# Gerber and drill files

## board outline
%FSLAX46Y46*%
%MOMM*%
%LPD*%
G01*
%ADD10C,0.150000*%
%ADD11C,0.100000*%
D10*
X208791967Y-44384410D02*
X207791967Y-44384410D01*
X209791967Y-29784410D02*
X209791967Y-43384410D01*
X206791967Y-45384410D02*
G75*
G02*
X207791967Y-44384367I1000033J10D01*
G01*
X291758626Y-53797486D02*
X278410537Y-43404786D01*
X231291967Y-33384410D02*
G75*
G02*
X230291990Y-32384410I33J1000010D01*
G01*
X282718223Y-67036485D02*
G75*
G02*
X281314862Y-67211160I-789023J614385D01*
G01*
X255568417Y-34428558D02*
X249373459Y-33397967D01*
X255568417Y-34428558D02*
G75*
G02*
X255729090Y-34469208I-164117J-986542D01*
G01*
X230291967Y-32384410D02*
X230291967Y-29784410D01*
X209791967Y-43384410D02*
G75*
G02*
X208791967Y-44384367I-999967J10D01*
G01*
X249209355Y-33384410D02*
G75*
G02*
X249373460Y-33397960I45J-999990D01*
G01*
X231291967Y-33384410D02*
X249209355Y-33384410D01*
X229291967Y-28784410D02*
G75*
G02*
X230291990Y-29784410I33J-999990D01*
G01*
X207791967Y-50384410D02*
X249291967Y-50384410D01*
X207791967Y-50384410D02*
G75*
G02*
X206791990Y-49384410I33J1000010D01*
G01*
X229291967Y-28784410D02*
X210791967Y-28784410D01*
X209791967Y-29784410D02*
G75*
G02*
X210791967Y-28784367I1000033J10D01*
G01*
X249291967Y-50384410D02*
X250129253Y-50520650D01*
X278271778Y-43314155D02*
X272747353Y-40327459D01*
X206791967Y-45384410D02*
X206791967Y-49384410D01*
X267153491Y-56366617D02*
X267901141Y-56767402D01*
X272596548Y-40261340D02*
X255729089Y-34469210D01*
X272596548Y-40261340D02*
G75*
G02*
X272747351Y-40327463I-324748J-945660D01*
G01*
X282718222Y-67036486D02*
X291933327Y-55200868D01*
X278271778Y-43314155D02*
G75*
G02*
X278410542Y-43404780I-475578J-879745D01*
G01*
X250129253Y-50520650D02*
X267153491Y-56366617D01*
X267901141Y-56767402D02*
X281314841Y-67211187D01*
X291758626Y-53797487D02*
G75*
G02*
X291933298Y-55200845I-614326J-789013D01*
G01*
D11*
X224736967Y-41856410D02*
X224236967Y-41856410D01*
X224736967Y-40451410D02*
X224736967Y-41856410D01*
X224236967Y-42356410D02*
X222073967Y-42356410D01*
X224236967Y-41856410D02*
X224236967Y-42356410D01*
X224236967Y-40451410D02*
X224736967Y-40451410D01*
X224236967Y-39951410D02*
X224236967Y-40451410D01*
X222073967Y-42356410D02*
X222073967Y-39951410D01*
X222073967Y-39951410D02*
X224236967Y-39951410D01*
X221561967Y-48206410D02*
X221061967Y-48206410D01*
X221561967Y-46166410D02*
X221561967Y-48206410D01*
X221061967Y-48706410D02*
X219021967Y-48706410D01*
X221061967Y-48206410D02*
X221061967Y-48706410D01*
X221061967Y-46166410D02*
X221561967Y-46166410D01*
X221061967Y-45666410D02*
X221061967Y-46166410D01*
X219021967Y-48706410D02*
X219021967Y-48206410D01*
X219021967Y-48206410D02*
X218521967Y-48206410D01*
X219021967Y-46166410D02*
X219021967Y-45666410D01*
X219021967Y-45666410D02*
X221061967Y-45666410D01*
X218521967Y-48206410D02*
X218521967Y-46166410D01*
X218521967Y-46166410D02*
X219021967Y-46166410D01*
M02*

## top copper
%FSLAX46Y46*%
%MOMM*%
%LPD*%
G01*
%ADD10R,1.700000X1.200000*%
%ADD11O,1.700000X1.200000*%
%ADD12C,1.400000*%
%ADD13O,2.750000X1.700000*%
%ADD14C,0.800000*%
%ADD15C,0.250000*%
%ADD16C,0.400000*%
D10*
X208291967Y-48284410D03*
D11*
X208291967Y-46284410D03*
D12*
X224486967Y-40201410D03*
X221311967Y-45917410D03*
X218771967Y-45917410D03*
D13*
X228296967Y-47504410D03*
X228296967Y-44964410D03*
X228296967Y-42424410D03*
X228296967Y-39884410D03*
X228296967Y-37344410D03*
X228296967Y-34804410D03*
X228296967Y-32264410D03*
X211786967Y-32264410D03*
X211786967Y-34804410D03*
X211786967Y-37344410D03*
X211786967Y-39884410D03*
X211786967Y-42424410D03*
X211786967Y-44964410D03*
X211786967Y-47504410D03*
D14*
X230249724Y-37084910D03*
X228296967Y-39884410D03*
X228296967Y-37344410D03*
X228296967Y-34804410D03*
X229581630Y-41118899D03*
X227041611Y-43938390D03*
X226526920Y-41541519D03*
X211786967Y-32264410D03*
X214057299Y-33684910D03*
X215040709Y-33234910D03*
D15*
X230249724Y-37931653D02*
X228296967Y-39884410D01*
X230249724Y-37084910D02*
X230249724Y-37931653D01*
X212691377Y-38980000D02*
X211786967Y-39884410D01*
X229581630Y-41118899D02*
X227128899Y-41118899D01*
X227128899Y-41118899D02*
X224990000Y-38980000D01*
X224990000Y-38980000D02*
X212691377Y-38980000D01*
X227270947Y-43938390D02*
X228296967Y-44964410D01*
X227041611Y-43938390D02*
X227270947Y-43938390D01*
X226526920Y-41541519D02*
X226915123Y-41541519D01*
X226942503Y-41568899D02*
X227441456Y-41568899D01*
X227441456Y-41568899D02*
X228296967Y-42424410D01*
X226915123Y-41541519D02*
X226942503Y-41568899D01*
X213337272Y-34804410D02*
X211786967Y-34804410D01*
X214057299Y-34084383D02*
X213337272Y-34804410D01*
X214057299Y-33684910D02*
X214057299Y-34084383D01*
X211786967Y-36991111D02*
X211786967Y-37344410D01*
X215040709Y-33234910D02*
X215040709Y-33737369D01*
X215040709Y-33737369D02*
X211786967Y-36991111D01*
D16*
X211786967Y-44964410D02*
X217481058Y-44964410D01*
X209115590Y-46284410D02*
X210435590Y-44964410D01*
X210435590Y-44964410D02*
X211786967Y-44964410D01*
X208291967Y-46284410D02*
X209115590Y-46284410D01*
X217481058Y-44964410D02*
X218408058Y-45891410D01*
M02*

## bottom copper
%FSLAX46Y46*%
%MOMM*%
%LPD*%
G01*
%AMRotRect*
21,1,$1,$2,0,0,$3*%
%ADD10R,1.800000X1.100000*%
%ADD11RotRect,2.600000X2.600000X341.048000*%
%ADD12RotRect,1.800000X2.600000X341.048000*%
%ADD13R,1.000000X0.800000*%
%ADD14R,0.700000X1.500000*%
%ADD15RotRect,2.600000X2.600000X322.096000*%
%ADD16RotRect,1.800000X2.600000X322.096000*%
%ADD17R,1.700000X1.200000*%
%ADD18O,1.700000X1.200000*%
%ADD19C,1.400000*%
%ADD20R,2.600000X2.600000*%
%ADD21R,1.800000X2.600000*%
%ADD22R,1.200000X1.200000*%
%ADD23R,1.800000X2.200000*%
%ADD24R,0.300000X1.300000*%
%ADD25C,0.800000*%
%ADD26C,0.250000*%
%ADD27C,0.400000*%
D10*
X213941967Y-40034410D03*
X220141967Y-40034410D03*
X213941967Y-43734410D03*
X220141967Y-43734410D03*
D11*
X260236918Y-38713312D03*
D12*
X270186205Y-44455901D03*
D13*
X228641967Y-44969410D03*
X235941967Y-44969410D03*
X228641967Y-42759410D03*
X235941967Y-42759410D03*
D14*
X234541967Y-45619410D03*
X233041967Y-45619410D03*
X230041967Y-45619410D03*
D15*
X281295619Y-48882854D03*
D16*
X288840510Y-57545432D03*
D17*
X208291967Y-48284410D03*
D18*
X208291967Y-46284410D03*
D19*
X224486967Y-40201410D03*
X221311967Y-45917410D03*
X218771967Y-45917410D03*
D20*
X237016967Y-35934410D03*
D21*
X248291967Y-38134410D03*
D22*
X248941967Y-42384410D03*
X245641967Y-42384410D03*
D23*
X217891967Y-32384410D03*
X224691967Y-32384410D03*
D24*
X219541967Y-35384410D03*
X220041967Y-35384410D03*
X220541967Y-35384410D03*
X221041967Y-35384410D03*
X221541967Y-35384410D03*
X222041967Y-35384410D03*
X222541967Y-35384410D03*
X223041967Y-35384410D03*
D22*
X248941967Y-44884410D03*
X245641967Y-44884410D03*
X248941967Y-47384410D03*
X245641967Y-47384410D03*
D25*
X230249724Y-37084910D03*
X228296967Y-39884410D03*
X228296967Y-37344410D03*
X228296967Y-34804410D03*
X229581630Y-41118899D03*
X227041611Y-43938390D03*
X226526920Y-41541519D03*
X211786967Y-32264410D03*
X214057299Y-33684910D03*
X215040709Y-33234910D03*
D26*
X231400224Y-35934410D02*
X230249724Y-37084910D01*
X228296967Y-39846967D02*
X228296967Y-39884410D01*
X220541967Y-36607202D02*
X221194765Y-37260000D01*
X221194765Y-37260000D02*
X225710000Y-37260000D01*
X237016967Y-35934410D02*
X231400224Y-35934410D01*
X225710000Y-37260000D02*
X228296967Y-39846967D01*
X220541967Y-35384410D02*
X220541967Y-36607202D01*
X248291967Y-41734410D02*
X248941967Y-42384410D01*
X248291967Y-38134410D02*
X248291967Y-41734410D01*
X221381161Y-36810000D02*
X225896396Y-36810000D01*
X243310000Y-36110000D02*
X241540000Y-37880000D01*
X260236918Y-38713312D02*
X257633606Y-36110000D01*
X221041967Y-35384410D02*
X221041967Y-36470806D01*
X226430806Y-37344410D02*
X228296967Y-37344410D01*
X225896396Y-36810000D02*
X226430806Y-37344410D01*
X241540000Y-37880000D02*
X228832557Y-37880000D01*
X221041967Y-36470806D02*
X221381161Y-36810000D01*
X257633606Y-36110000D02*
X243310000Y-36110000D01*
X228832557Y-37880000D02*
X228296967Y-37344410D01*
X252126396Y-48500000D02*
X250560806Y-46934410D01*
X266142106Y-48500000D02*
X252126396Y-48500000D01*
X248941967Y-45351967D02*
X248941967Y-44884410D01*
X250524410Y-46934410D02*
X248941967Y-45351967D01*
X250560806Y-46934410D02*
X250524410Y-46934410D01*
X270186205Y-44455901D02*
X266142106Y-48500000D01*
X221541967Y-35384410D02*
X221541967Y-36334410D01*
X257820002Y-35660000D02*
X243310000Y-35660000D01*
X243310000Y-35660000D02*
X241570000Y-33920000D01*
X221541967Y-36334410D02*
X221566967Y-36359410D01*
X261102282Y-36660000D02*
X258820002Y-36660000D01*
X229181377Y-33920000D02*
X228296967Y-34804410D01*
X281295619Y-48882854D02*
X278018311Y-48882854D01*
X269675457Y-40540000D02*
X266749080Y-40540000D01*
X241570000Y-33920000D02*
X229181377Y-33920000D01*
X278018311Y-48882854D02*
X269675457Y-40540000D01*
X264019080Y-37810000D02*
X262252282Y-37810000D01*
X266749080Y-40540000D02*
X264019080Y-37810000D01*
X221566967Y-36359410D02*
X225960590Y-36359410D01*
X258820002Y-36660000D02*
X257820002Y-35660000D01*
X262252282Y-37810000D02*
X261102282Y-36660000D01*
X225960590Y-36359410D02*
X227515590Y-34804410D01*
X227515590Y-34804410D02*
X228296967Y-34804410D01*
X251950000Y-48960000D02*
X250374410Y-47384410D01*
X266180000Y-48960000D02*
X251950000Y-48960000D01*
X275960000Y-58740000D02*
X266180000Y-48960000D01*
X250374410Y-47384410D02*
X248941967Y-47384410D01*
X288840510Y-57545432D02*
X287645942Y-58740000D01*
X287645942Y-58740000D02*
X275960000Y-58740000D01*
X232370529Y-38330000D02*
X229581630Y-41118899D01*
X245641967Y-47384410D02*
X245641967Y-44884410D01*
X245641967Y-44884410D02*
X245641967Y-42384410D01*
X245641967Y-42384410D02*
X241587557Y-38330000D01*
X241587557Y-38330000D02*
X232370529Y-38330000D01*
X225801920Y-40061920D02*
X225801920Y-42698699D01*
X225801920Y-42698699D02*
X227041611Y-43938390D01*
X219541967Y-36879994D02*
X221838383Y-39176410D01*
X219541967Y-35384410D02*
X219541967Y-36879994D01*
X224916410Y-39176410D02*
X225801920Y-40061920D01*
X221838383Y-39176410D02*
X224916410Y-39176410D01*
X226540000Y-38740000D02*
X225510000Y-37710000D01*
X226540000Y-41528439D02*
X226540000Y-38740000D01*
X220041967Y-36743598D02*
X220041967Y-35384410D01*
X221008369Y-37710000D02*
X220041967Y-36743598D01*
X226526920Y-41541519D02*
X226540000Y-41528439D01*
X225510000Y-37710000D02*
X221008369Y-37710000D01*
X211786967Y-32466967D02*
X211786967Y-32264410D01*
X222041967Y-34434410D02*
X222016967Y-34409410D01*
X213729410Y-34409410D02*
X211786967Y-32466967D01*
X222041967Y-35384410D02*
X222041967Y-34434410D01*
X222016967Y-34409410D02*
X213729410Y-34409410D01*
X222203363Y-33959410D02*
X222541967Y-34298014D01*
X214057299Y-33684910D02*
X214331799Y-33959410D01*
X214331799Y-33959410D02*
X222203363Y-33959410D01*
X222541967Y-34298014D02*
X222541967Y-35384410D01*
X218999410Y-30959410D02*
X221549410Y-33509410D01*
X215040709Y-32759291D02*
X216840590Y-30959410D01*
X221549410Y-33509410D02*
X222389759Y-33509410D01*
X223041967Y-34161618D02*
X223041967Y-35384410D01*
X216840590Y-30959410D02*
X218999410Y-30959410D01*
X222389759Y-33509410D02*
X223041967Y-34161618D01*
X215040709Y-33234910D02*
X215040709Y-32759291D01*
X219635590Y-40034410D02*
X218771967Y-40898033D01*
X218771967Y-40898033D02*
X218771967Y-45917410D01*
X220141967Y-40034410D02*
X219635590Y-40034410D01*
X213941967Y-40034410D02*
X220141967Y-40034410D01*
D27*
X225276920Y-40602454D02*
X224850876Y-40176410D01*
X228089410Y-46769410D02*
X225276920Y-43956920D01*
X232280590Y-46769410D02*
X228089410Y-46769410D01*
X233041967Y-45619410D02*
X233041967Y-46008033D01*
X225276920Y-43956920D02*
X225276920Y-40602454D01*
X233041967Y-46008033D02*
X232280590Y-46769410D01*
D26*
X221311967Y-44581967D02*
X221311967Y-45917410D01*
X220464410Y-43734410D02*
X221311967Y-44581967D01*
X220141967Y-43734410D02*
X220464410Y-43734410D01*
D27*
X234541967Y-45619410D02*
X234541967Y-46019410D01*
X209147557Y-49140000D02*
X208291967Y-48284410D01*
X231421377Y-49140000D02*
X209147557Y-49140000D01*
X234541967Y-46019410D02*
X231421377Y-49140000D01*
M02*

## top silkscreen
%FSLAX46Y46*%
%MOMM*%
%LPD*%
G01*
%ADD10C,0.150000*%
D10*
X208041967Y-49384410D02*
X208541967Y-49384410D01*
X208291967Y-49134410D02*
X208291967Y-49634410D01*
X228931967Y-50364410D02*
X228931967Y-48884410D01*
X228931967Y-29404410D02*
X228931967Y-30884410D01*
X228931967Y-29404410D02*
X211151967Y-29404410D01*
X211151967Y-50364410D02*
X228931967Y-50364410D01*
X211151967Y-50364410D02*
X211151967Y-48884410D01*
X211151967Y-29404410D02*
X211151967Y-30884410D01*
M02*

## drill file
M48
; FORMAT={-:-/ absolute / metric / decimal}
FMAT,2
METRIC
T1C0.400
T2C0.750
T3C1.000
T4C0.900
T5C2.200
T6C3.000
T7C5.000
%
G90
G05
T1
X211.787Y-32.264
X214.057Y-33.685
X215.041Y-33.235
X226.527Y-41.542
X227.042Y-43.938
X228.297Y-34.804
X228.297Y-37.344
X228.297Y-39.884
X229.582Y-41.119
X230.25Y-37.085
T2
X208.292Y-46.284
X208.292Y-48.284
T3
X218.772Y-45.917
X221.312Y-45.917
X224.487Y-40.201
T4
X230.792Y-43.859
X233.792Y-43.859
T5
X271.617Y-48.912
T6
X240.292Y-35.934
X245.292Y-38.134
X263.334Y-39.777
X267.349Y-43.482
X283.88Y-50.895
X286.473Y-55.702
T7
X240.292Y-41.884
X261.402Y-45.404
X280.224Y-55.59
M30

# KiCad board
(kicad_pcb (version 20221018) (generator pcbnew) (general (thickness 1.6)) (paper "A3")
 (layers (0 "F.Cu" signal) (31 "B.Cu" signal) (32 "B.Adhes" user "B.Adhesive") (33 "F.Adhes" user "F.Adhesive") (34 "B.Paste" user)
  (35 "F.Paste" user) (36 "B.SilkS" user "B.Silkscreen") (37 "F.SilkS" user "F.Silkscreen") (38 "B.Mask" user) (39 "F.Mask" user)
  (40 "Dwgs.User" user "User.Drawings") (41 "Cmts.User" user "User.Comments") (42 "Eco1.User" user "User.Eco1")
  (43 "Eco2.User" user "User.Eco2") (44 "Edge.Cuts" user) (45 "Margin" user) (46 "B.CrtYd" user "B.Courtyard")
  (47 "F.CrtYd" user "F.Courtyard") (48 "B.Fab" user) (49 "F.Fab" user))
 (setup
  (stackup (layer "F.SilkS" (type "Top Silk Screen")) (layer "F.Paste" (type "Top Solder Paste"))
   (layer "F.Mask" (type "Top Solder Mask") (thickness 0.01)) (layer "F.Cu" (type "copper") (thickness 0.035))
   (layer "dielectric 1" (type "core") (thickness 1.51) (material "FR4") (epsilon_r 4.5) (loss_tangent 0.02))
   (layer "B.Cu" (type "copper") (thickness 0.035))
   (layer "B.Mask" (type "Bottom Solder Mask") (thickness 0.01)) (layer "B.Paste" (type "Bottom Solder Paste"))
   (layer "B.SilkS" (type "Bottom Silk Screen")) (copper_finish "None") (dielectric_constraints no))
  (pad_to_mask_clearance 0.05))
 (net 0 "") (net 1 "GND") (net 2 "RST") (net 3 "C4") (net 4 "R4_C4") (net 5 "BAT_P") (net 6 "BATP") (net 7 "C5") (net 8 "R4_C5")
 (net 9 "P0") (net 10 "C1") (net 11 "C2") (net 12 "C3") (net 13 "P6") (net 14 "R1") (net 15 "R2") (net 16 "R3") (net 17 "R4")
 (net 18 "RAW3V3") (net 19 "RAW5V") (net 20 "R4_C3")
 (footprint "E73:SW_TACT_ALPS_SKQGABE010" (layer "F.Cu") (at 217.041967 41.88441)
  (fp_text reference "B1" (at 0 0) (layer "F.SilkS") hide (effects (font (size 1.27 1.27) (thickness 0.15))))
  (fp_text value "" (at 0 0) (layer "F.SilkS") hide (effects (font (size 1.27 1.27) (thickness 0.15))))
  (pad "1" smd rect (at -3.1 -1.85) (size 1.8 1.1) (layers "B.Cu" "B.Paste" "B.Mask") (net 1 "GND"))
  (pad "1" smd rect (at 3.1 -1.85) (size 1.8 1.1) (layers "B.Cu" "B.Paste" "B.Mask") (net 1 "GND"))
  (pad "2" smd rect (at -3.1 1.85) (size 1.8 1.1) (layers "B.Cu" "B.Paste" "B.Mask") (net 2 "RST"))
  (pad "2" smd rect (at 3.1 1.85) (size 1.8 1.1) (layers "B.Cu" "B.Paste" "B.Mask") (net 2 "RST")))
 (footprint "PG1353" (layer "F.Cu") (at 261.401967 45.40441 -18.952)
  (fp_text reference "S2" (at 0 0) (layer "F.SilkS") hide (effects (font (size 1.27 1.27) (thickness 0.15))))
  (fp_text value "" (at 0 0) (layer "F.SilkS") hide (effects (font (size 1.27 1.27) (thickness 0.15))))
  (pad "" np_thru_hole circle (at 0 -5.95) (size 3 3) (drill 3) (layers "*.Cu" "*.Mask"))
  (pad "" np_thru_hole circle (at 0 0) (size 5 5) (drill 5) (layers "*.Cu" "*.Mask"))
  (pad "" np_thru_hole circle (at 5 -3.75) (size 3 3) (drill 3) (layers "*.Cu" "*.Mask"))
  (pad "1" smd rect (at -3.275 -5.95 341.048) (size 2.6 2.6) (layers "B.Cu" "B.Paste" "B.Mask") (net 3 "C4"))
  (pad "2" smd rect (at 8 -3.75 341.048) (size 1.8 2.6) (layers "B.Cu" "B.Paste" "B.Mask") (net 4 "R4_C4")))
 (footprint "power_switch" (layer "F.Cu") (at 232.291967 43.88441 90)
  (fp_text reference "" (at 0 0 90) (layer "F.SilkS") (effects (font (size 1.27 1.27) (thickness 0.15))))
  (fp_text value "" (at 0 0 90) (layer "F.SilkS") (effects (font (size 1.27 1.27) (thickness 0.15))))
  (pad "" smd rect (at -1.085 -3.65) (size 1 0.8) (layers "B.Cu" "B.Paste" "B.Mask"))
  (pad "" smd rect (at -1.085 3.65) (size 1 0.8) (layers "B.Cu" "B.Paste" "B.Mask"))
  (pad "" np_thru_hole circle (at 0.025 -1.5 180) (size 0.9 0.9) (drill 0.9) (layers "*.Cu" "*.Mask"))
  (pad "" np_thru_hole circle (at 0.025 1.5 180) (size 0.9 0.9) (drill 0.9) (layers "*.Cu" "*.Mask"))
  (pad "" smd rect (at 1.125 -3.65) (size 1 0.8) (layers "B.Cu" "B.Paste" "B.Mask"))
  (pad "" smd rect (at 1.125 3.65) (size 1 0.8) (layers "B.Cu" "B.Paste" "B.Mask"))
  (pad "4" smd rect (at -1.735 2.25) (size 0.7 1.5) (layers "B.Cu" "B.Paste" "B.Mask") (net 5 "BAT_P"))
  (pad "5" smd rect (at -1.735 0.75) (size 0.7 1.5) (layers "B.Cu" "B.Paste" "B.Mask") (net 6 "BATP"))
  (pad "6" smd rect (at -1.735 -2.25) (size 0.7 1.5) (layers "B.Cu" "B.Paste" "B.Mask")))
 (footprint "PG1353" (layer "F.Cu") (at 280.224404 55.589614 -37.904)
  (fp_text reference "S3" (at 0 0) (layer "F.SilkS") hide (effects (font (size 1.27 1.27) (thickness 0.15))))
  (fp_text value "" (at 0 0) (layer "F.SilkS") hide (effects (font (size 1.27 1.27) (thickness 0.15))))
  (pad "" np_thru_hole circle (at 0 -5.95) (size 3 3) (drill 3) (layers "*.Cu" "*.Mask"))
  (pad "" np_thru_hole circle (at 0 0) (size 5 5) (drill 5) (layers "*.Cu" "*.Mask"))
  (pad "" np_thru_hole circle (at 5 -3.75) (size 3 3) (drill 3) (layers "*.Cu" "*.Mask"))
  (pad "1" smd rect (at -3.275 -5.95 322.096) (size 2.6 2.6) (layers "B.Cu" "B.Paste" "B.Mask") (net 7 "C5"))
  (pad "2" smd rect (at 8 -3.75 322.096) (size 1.8 2.6) (layers "B.Cu" "B.Paste" "B.Mask") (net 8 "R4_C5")))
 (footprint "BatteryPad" (layer "F.Cu") (at 208.291967 47.28441 90)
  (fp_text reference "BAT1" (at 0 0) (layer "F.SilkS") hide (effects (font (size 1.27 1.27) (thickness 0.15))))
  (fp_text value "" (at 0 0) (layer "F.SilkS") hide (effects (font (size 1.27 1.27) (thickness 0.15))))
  (fp_line (start -2.1 -0.25) (end -2.1 0.25) (stroke (width 0.15) (type solid)) (layer "F.SilkS"))
  (fp_line (start -1.85 0) (end -2.35 0) (stroke (width 0.15) (type solid)) (layer "F.SilkS"))
  (pad "1" thru_hole rect (at -1 0 90) (size 1.2 1.7) (drill 0.75) (layers "*.Cu" "*.Mask") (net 5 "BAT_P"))
  (pad "2" thru_hole oval (at 1 0 90) (size 1.2 1.7) (drill 0.75) (layers "*.Cu" "*.Mask") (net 1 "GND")))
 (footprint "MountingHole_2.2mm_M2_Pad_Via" (layer "F.Cu") (at 271.61651 48.91199 -18.952)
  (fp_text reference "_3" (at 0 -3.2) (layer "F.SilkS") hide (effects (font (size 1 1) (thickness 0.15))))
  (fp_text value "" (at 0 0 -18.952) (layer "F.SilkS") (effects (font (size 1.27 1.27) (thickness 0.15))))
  (pad "" np_thru_hole circle (at 0 0) (size 2.2 2.2) (drill 2.2) (layers "*.Cu" "*.Mask")))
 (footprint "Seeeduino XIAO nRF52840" (layer "F.Cu") (at 220.041967 39.88441 180)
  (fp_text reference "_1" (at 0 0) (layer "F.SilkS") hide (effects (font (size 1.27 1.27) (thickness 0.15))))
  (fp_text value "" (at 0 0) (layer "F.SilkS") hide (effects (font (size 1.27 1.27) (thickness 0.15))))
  (fp_line (start -8.89 -10.48) (end -8.89 -9) (stroke (width 0.15) (type solid)) (layer "F.SilkS"))
  (fp_line (start -8.89 10.48) (end -8.89 9) (stroke (width 0.15) (type solid)) (layer "F.SilkS"))
  (fp_line (start -8.89 10.48) (end 8.89 10.48) (stroke (width 0.15) (type solid)) (layer "F.SilkS"))
  (fp_line (start 8.89 -10.48) (end -8.89 -10.48) (stroke (width 0.15) (type solid)) (layer "F.SilkS"))
  (fp_line (start 8.89 -10.48) (end 8.89 -9) (stroke (width 0.15) (type solid)) (layer "F.SilkS"))
  (fp_line (start 8.89 10.48) (end 8.89 9) (stroke (width 0.15) (type solid)) (layer "F.SilkS"))
  (fp_line (start -4.695 -1.972) (end -4.195 -1.972) (stroke (width 0.1) (type solid)) (layer "Edge.Cuts"))
  (fp_line (start -4.695 -0.567) (end -4.695 -1.972) (stroke (width 0.1) (type solid)) (layer "Edge.Cuts"))
  (fp_line (start -4.195 -2.472) (end -2.032 -2.472) (stroke (width 0.1) (type solid)) (layer "Edge.Cuts"))
  (fp_line (start -4.195 -1.972) (end -4.195 -2.472) (stroke (width 0.1) (type solid)) (layer "Edge.Cuts"))
  (fp_line (start -4.195 -0.567) (end -4.695 -0.567) (stroke (width 0.1) (type solid)) (layer "Edge.Cuts"))
  (fp_line (start -4.195 -0.067) (end -4.195 -0.567) (stroke (width 0.1) (type solid)) (layer "Edge.Cuts"))
  (fp_line (start -2.032 -2.472) (end -2.032 -0.067) (stroke (width 0.1) (type solid)) (layer "Edge.Cuts"))
  (fp_line (start -2.032 -0.067) (end -4.195 -0.067) (stroke (width 0.1) (type solid)) (layer "Edge.Cuts"))
  (fp_line (start -1.52 -8.322) (end -1.02 -8.322) (stroke (width 0.1) (type solid)) (layer "Edge.Cuts"))
  (fp_line (start -1.52 -6.282) (end -1.52 -8.322) (stroke (width 0.1) (type solid)) (layer "Edge.Cuts"))
  (fp_line (start -1.02 -8.822) (end 1.02 -8.822) (stroke (width 0.1) (type solid)) (layer "Edge.Cuts"))
  (fp_line (start -1.02 -8.322) (end -1.02 -8.822) (stroke (width 0.1) (type solid)) (layer "Edge.Cuts"))
  (fp_line (start -1.02 -6.282) (end -1.52 -6.282) (stroke (width 0.1) (type solid)) (layer "Edge.Cuts"))
  (fp_line (start -1.02 -5.782) (end -1.02 -6.282) (stroke (width 0.1) (type solid)) (layer "Edge.Cuts"))
  (fp_line (start 1.02 -8.822) (end 1.02 -8.322) (stroke (width 0.1) (type solid)) (layer "Edge.Cuts"))
  (fp_line (start 1.02 -8.322) (end 1.52 -8.322) (stroke (width 0.1) (type solid)) (layer "Edge.Cuts"))
  (fp_line (start 1.02 -6.282) (end 1.02 -5.782) (stroke (width 0.1) (type solid)) (layer "Edge.Cuts"))
  (fp_line (start 1.02 -5.782) (end -1.02 -5.782) (stroke (width 0.1) (type solid)) (layer "Edge.Cuts"))
  (fp_line (start 1.52 -8.322) (end 1.52 -6.282) (stroke (width 0.1) (type solid)) (layer "Edge.Cuts"))
  (fp_line (start 1.52 -6.282) (end 1.02 -6.282) (stroke (width 0.1) (type solid)) (layer "Edge.Cuts"))
  (pad "" thru_hole circle (at -4.445 -0.317) (size 1.4 1.4) (drill 1) (layers "*.Cu" "*.Mask") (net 6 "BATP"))
  (pad "" thru_hole circle (at -1.27 -6.033) (size 1.4 1.4) (drill 1) (layers "*.Cu" "*.Mask") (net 2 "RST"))
  (pad "" thru_hole circle (at 1.27 -6.033) (size 1.4 1.4) (drill 1) (layers "*.Cu" "*.Mask") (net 1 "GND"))
  (pad "1" smd oval (at -8.255 -7.62 180) (size 2.75 1.7) (layers "F.Cu" "F.Paste" "F.Mask") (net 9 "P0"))
  (pad "2" smd oval (at -8.255 -5.08 180) (size 2.75 1.7) (layers "F.Cu" "F.Paste" "F.Mask") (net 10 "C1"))
  (pad "3" smd oval (at -8.255 -2.54 180) (size 2.75 1.7) (layers "F.Cu" "F.Paste" "F.Mask") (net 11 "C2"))
  (pad "4" smd oval (at -8.255 0 180) (size 2.75 1.7) (layers "F.Cu" "F.Paste" "F.Mask") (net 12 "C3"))
  (pad "5" smd oval (at -8.255 2.54 180) (size 2.75 1.7) (layers "F.Cu" "F.Paste" "F.Mask") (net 3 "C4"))
  (pad "6" smd oval (at -8.255 5.08 180) (size 2.75 1.7) (layers "F.Cu" "F.Paste" "F.Mask") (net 7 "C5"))
  (pad "7" smd oval (at -8.255 7.62 180) (size 2.75 1.7) (layers "F.Cu" "F.Paste" "F.Mask") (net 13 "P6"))
  (pad "8" smd oval (at 8.255 7.62 180) (size 2.75 1.7) (layers "F.Cu" "F.Paste" "F.Mask") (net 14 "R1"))
  (pad "9" smd oval (at 8.255 5.08 180) (size 2.75 1.7) (layers "F.Cu" "F.Paste" "F.Mask") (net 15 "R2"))
  (pad "10" smd oval (at 8.255 2.54 180) (size 2.75 1.7) (layers "F.Cu" "F.Paste" "F.Mask") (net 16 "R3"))
  (pad "11" smd oval (at 8.255 0 180) (size 2.75 1.7) (layers "F.Cu" "F.Paste" "F.Mask") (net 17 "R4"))
  (pad "12" smd oval (at 8.255 -2.54 180) (size 2.75 1.7) (layers "F.Cu" "F.Paste" "F.Mask") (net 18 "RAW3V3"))
  (pad "13" smd oval (at 8.255 -5.08 180) (size 2.75 1.7) (layers "F.Cu" "F.Paste" "F.Mask") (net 1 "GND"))
  (pad "14" smd oval (at 8.255 -7.62 180) (size 2.75 1.7) (layers "F.Cu" "F.Paste" "F.Mask") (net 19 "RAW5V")))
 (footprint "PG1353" (layer "F.Cu") (at 240.291967 41.88441)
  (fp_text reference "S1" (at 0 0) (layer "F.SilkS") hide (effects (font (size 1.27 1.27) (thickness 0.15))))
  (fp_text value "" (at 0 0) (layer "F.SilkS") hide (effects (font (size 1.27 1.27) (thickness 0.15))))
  (pad "" np_thru_hole circle (at 0 -5.95) (size 3 3) (drill 3) (layers "*.Cu" "*.Mask"))
  (pad "" np_thru_hole circle (at 0 0) (size 5 5) (drill 5) (layers "*.Cu" "*.Mask"))
  (pad "" np_thru_hole circle (at 5 -3.75) (size 3 3) (drill 3) (layers "*.Cu" "*.Mask"))
  (pad "1" smd rect (at -3.275 -5.95) (size 2.6 2.6) (layers "B.Cu" "B.Paste" "B.Mask") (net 12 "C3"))
  (pad "2" smd rect (at 8 -3.75) (size 1.8 2.6) (layers "B.Cu" "B.Paste" "B.Mask") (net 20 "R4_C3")))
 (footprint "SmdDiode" (layer "B.Cu") (at 247.291967 44.88441 -90)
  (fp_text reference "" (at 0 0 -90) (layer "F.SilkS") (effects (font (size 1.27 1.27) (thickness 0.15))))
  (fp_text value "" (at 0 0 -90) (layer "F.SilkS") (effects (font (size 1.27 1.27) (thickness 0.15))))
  (pad "1" smd rect (at -2.5 -1.65 270) (size 1.2 1.2) (layers "B.Cu" "B.Paste" "B.Mask") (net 20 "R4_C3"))
  (pad "2" smd rect (at -2.5 1.65 270) (size 1.2 1.2) (layers "B.Cu" "B.Paste" "B.Mask") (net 17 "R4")))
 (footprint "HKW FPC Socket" (layer "B.Cu") (at 221.291967 32.38441)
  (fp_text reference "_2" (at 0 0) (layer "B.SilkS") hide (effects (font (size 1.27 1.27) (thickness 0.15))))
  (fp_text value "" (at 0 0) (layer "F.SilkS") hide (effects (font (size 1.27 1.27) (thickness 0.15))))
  (pad "" smd rect (at -3.4 0) (size 1.8 2.2) (layers "B.Cu" "B.Paste" "B.Mask"))
  (pad "" smd rect (at 3.4 0) (size 1.8 2.2) (layers "B.Cu" "B.Paste" "B.Mask"))
  (pad "1" smd rect (at -1.75 3) (size 0.3 1.3) (layers "B.Cu" "B.Paste" "B.Mask") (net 10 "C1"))
  (pad "2" smd rect (at -1.25 3) (size 0.3 1.3) (layers "B.Cu" "B.Paste" "B.Mask") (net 11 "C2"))
  (pad "3" smd rect (at -0.75 3) (size 0.3 1.3) (layers "B.Cu" "B.Paste" "B.Mask") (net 12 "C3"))
  (pad "4" smd rect (at -0.25 3) (size 0.3 1.3) (layers "B.Cu" "B.Paste" "B.Mask") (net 3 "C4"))
  (pad "5" smd rect (at 0.25 3) (size 0.3 1.3) (layers "B.Cu" "B.Paste" "B.Mask") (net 7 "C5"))
  (pad "6" smd rect (at 0.75 3) (size 0.3 1.3) (layers "B.Cu" "B.Paste" "B.Mask") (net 14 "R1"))
  (pad "7" smd rect (at 1.25 3) (size 0.3 1.3) (layers "B.Cu" "B.Paste" "B.Mask") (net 15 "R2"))
  (pad "8" smd rect (at 1.75 3) (size 0.3 1.3) (layers "B.Cu" "B.Paste" "B.Mask") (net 16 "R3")))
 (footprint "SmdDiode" (layer "B.Cu") (at 247.291967 44.88441 -90)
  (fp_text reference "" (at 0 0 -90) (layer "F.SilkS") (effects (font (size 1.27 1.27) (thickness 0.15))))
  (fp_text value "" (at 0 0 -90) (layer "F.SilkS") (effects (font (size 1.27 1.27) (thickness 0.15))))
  (pad "1" smd rect (at 0 -1.65 270) (size 1.2 1.2) (layers "B.Cu" "B.Paste" "B.Mask") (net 4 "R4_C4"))
  (pad "2" smd rect (at 0 1.65 270) (size 1.2 1.2) (layers "B.Cu" "B.Paste" "B.Mask") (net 17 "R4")))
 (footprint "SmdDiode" (layer "B.Cu") (at 247.291967 44.88441 -90)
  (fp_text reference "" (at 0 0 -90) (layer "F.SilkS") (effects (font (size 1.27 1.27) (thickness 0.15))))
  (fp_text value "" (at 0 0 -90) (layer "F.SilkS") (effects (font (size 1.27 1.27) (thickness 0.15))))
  (pad "1" smd rect (at 2.5 -1.65 270) (size 1.2 1.2) (layers "B.Cu" "B.Paste" "B.Mask") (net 8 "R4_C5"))
  (pad "2" smd rect (at 2.5 1.65 270) (size 1.2 1.2) (layers "B.Cu" "B.Paste" "B.Mask") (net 17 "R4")))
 (gr_line (start 208.791967 44.38441) (end 207.791967 44.38441) (stroke (width 0.15) (type solid)) (layer "Edge.Cuts"))
 (gr_line (start 209.791967 29.78441) (end 209.791967 43.38441) (stroke (width 0.15) (type solid)) (layer "Edge.Cuts"))
 (gr_arc (start 206.791967 45.38441) (mid 207.08486 44.677303) (end 207.791967 44.38441) (stroke (width 0.15) (type solid))
  (layer "Edge.Cuts"))
 (gr_line (start 291.758626 53.797486) (end 278.410537 43.404786) (stroke (width 0.15) (type solid)) (layer "Edge.Cuts"))
 (gr_arc (start 231.291967 33.38441) (mid 230.58486 33.091517) (end 230.291967 32.38441) (stroke (width 0.15) (type solid))
  (layer "Edge.Cuts"))
 (gr_arc (start 282.718223 67.036485) (mid 282.052714 67.414486) (end 281.314841 67.211187) (stroke (width 0.15) (type solid))
  (layer "Edge.Cuts"))
 (gr_line (start 255.568417 34.428558) (end 249.373459 33.397967) (stroke (width 0.15) (type solid)) (layer "Edge.Cuts"))
 (gr_arc (start 255.568417 34.428558) (mid 255.649597 34.44555) (end 255.729089 34.46921) (stroke (width 0.15) (type solid))
  (layer "Edge.Cuts"))
 (gr_line (start 230.291967 32.38441) (end 230.291967 29.78441) (stroke (width 0.15) (type solid)) (layer "Edge.Cuts"))
 (gr_arc (start 209.791967 43.38441) (mid 209.499074 44.091517) (end 208.791967 44.38441) (stroke (width 0.15) (type solid))
  (layer "Edge.Cuts"))
 (gr_arc (start 249.209355 33.38441) (mid 249.291687 33.387805) (end 249.373459 33.397967) (stroke (width 0.15) (type solid))
  (layer "Edge.Cuts"))
 (gr_line (start 231.291967 33.38441) (end 249.209355 33.38441) (stroke (width 0.15) (type solid)) (layer "Edge.Cuts"))
 (gr_arc (start 229.291967 28.78441) (mid 229.999074 29.077303) (end 230.291967 29.78441) (stroke (width 0.15) (type solid))
  (layer "Edge.Cuts"))
 (gr_line (start 207.791967 50.38441) (end 249.291967 50.38441) (stroke (width 0.15) (type solid)) (layer "Edge.Cuts"))
 (gr_arc (start 207.791967 50.38441) (mid 207.08486 50.091517) (end 206.791967 49.38441) (stroke (width 0.15) (type solid))
  (layer "Edge.Cuts"))
 (gr_line (start 229.291967 28.78441) (end 210.791967 28.78441) (stroke (width 0.15) (type solid)) (layer "Edge.Cuts"))
 (gr_arc (start 209.791967 29.78441) (mid 210.08486 29.077303) (end 210.791967 28.78441) (stroke (width 0.15) (type solid))
  (layer "Edge.Cuts"))
 (gr_line (start 249.291967 50.38441) (end 250.129253 50.52065) (stroke (width 0.15) (type solid)) (layer "Edge.Cuts"))
 (gr_line (start 278.271778 43.314155) (end 272.747353 40.327459) (stroke (width 0.15) (type solid)) (layer "Edge.Cuts"))
 (gr_line (start 206.791967 45.38441) (end 206.791967 49.38441) (stroke (width 0.15) (type solid)) (layer "Edge.Cuts"))
 (gr_line (start 267.153491 56.366617) (end 267.901141 56.767402) (stroke (width 0.15) (type solid)) (layer "Edge.Cuts"))
 (gr_line (start 272.596548 40.26134) (end 255.729089 34.46921) (stroke (width 0.15) (type solid)) (layer "Edge.Cuts"))
 (gr_arc (start 272.596548 40.26134) (mid 272.673314 40.29129) (end 272.747353 40.327459) (stroke (width 0.15) (type solid))
  (layer "Edge.Cuts"))
 (gr_line (start 282.718222 67.036486) (end 291.933327 55.200868) (stroke (width 0.15) (type solid)) (layer "Edge.Cuts"))
 (gr_arc (start 278.271778 43.314155) (mid 278.343038 43.356591) (end 278.410537 43.404786) (stroke (width 0.15) (type solid))
  (layer "Edge.Cuts"))
 (gr_line (start 250.129253 50.52065) (end 267.153491 56.366617) (stroke (width 0.15) (type solid)) (layer "Edge.Cuts"))
 (gr_line (start 267.901141 56.767402) (end 281.314841 67.211187) (stroke (width 0.15) (type solid)) (layer "Edge.Cuts"))
 (gr_arc (start 291.758626 53.797487) (mid 292.136626 54.462996) (end 291.933327 55.200868) (stroke (width 0.15) (type solid))
  (layer "Edge.Cuts"))
 (segment (start 230.249724 37.931653) (end 228.296967 39.88441) (width 0.25) (layer "F.Cu") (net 12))
 (segment (start 230.249724 37.08491) (end 230.249724 37.931653) (width 0.25) (layer "F.Cu") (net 12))
 (via (at 230.249724 37.08491) (size 0.8) (drill 0.4) (layers "F.Cu" "B.Cu") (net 12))
 (via (at 228.296967 39.88441) (size 0.8) (drill 0.4) (layers "F.Cu" "B.Cu") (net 12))
 (segment (start 231.400224 35.93441) (end 230.249724 37.08491) (width 0.25) (layer "B.Cu") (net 12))
 (segment (start 228.296967 39.846967) (end 228.296967 39.88441) (width 0.25) (layer "B.Cu") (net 12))
 (segment (start 220.541967 36.607202) (end 221.194765 37.26) (width 0.25) (layer "B.Cu") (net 12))
 (segment (start 221.194765 37.26) (end 225.71 37.26) (width 0.25) (layer "B.Cu") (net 12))
 (segment (start 237.016967 35.93441) (end 231.400224 35.93441) (width 0.25) (layer "B.Cu") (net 12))
 (segment (start 225.71 37.26) (end 228.296967 39.846967) (width 0.25) (layer "B.Cu") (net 12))
 (segment (start 220.541967 35.38441) (end 220.541967 36.607202) (width 0.25) (layer "B.Cu") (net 12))
 (segment (start 248.291967 41.73441) (end 248.941967 42.38441) (width 0.25) (layer "B.Cu") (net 20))
 (segment (start 248.291967 38.13441) (end 248.291967 41.73441) (width 0.25) (layer "B.Cu") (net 20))
 (via (at 228.296967 37.34441) (size 0.8) (drill 0.4) (layers "F.Cu" "B.Cu") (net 3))
 (segment (start 221.381161 36.81) (end 225.896396 36.81) (width 0.25) (layer "B.Cu") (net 3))
 (segment (start 243.31 36.11) (end 241.54 37.88) (width 0.25) (layer "B.Cu") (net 3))
 (segment (start 260.236918 38.713312) (end 257.633606 36.11) (width 0.25) (layer "B.Cu") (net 3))
 (segment (start 221.041967 35.38441) (end 221.041967 36.470806) (width 0.25) (layer "B.Cu") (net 3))
 (segment (start 226.430806 37.34441) (end 228.296967 37.34441) (width 0.25) (layer "B.Cu") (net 3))
 (segment (start 225.896396 36.81) (end 226.430806 37.34441) (width 0.25) (layer "B.Cu") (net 3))
 (segment (start 241.54 37.88) (end 228.832557 37.88) (width 0.25) (layer "B.Cu") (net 3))
 (segment (start 221.041967 36.470806) (end 221.381161 36.81) (width 0.25) (layer "B.Cu") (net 3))
 (segment (start 257.633606 36.11) (end 243.31 36.11) (width 0.25) (layer "B.Cu") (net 3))
 (segment (start 228.832557 37.88) (end 228.296967 37.34441) (width 0.25) (layer "B.Cu") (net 3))
 (segment (start 252.126396 48.5) (end 250.560806 46.93441) (width 0.25) (layer "B.Cu") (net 4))
 (segment (start 266.142106 48.5) (end 252.126396 48.5) (width 0.25) (layer "B.Cu") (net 4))
 (segment (start 248.941967 45.351967) (end 248.941967 44.88441) (width 0.25) (layer "B.Cu") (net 4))
 (segment (start 250.52441 46.93441) (end 248.941967 45.351967) (width 0.25) (layer "B.Cu") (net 4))
 (segment (start 250.560806 46.93441) (end 250.52441 46.93441) (width 0.25) (layer "B.Cu") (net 4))
 (segment (start 270.186205 44.455901) (end 266.142106 48.5) (width 0.25) (layer "B.Cu") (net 4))
 (via (at 228.296967 34.80441) (size 0.8) (drill 0.4) (layers "F.Cu" "B.Cu") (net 7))
 (segment (start 221.541967 35.38441) (end 221.541967 36.33441) (width 0.25) (layer "B.Cu") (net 7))
 (segment (start 257.820002 35.66) (end 243.31 35.66) (width 0.25) (layer "B.Cu") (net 7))
 (segment (start 243.31 35.66) (end 241.57 33.92) (width 0.25) (layer "B.Cu") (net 7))
 (segment (start 221.541967 36.33441) (end 221.566967 36.35941) (width 0.25) (layer "B.Cu") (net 7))
 (segment (start 261.102282 36.66) (end 258.820002 36.66) (width 0.25) (layer "B.Cu") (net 7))
 (segment (start 229.181377 33.92) (end 228.296967 34.80441) (width 0.25) (layer "B.Cu") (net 7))
 (segment (start 281.295619 48.882854) (end 278.018311 48.882854) (width 0.25) (layer "B.Cu") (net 7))
 (segment (start 269.675457 40.54) (end 266.74908 40.54) (width 0.25) (layer "B.Cu") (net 7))
 (segment (start 241.57 33.92) (end 229.181377 33.92) (width 0.25) (layer "B.Cu") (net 7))
 (segment (start 278.018311 48.882854) (end 269.675457 40.54) (width 0.25) (layer "B.Cu") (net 7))
 (segment (start 264.01908 37.81) (end 262.252282 37.81) (width 0.25) (layer "B.Cu") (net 7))
 (segment (start 266.74908 40.54) (end 264.01908 37.81) (width 0.25) (layer "B.Cu") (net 7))
 (segment (start 221.566967 36.35941) (end 225.96059 36.35941) (width 0.25) (layer "B.Cu") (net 7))
 (segment (start 258.820002 36.66) (end 257.820002 35.66) (width 0.25) (layer "B.Cu") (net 7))
 (segment (start 262.252282 37.81) (end 261.102282 36.66) (width 0.25) (layer "B.Cu") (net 7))
 (segment (start 225.96059 36.35941) (end 227.51559 34.80441) (width 0.25) (layer "B.Cu") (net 7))
 (segment (start 227.51559 34.80441) (end 228.296967 34.80441) (width 0.25) (layer "B.Cu") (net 7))
 (segment (start 251.95 48.96) (end 250.37441 47.38441) (width 0.25) (layer "B.Cu") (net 8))
 (segment (start 266.18 48.96) (end 251.95 48.96) (width 0.25) (layer "B.Cu") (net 8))
 (segment (start 275.96 58.74) (end 266.18 48.96) (width 0.25) (layer "B.Cu") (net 8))
 (segment (start 250.37441 47.38441) (end 248.941967 47.38441) (width 0.25) (layer "B.Cu") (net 8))
 (segment (start 288.84051 57.545432) (end 287.645942 58.74) (width 0.25) (layer "B.Cu") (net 8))
 (segment (start 287.645942 58.74) (end 275.96 58.74) (width 0.25) (layer "B.Cu") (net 8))
 (segment (start 212.691377 38.98) (end 211.786967 39.88441) (width 0.25) (layer "F.Cu") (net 17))
 (segment (start 229.58163 41.118899) (end 227.128899 41.118899) (width 0.25) (layer "F.Cu") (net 17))
 (segment (start 227.128899 41.118899) (end 224.99 38.98) (width 0.25) (layer "F.Cu") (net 17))
 (segment (start 224.99 38.98) (end 212.691377 38.98) (width 0.25) (layer "F.Cu") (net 17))
 (via (at 229.58163 41.118899) (size 0.8) (drill 0.4) (layers "F.Cu" "B.Cu") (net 17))
 (segment (start 232.370529 38.33) (end 229.58163 41.118899) (width 0.25) (layer "B.Cu") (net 17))
 (segment (start 245.641967 47.38441) (end 245.641967 44.88441) (width 0.25) (layer "B.Cu") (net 17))
 (segment (start 245.641967 44.88441) (end 245.641967 42.38441) (width 0.25) (layer "B.Cu") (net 17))
 (segment (start 245.641967 42.38441) (end 241.587557 38.33) (width 0.25) (layer "B.Cu") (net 17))
 (segment (start 241.587557 38.33) (end 232.370529 38.33) (width 0.25) (layer "B.Cu") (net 17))
 (segment (start 227.270947 43.93839) (end 228.296967 44.96441) (width 0.25) (layer "F.Cu") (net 10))
 (segment (start 227.041611 43.93839) (end 227.270947 43.93839) (width 0.25) (layer "F.Cu") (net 10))
 (via (at 227.041611 43.93839) (size 0.8) (drill 0.4) (layers "F.Cu" "B.Cu") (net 10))
 (segment (start 225.80192 40.06192) (end 225.80192 42.698699) (width 0.25) (layer "B.Cu") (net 10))
 (segment (start 225.80192 42.698699) (end 227.041611 43.93839) (width 0.25) (layer "B.Cu") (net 10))
 (segment (start 219.541967 36.879994) (end 221.838383 39.17641) (width 0.25) (layer "B.Cu") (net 10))
 (segment (start 219.541967 35.38441) (end 219.541967 36.879994) (width 0.25) (layer "B.Cu") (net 10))
 (segment (start 224.91641 39.17641) (end 225.80192 40.06192) (width 0.25) (layer "B.Cu") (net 10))
 (segment (start 221.838383 39.17641) (end 224.91641 39.17641) (width 0.25) (layer "B.Cu") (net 10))
 (segment (start 226.52692 41.541519) (end 226.915123 41.541519) (width 0.25) (layer "F.Cu") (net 11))
 (segment (start 226.942503 41.568899) (end 227.441456 41.568899) (width 0.25) (layer "F.Cu") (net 11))
 (segment (start 227.441456 41.568899) (end 228.296967 42.42441) (width 0.25) (layer "F.Cu") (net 11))
 (segment (start 226.915123 41.541519) (end 226.942503 41.568899) (width 0.25) (layer "F.Cu") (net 11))
 (via (at 226.52692 41.541519) (size 0.8) (drill 0.4) (layers "F.Cu" "B.Cu") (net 11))
 (segment (start 226.54 38.74) (end 225.51 37.71) (width 0.25) (layer "B.Cu") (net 11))
 (segment (start 226.54 41.528439) (end 226.54 38.74) (width 0.25) (layer "B.Cu") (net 11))
 (segment (start 220.041967 36.743598) (end 220.041967 35.38441) (width 0.25) (layer "B.Cu") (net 11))
 (segment (start 221.008369 37.71) (end 220.041967 36.743598) (width 0.25) (layer "B.Cu") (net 11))
 (segment (start 226.52692 41.541519) (end 226.54 41.528439) (width 0.25) (layer "B.Cu") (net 11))
 (segment (start 225.51 37.71) (end 221.008369 37.71) (width 0.25) (layer "B.Cu") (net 11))
 (via (at 211.786967 32.26441) (size 0.8) (drill 0.4) (layers "F.Cu" "B.Cu") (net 14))
 (segment (start 211.786967 32.466967) (end 211.786967 32.26441) (width 0.25) (layer "B.Cu") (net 14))
 (segment (start 222.041967 34.43441) (end 222.016967 34.40941) (width 0.25) (layer "B.Cu") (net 14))
 (segment (start 213.72941 34.40941) (end 211.786967 32.466967) (width 0.25) (layer "B.Cu") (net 14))
 (segment (start 222.041967 35.38441) (end 222.041967 34.43441) (width 0.25) (layer "B.Cu") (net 14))
 (segment (start 222.016967 34.40941) (end 213.72941 34.40941) (width 0.25) (layer "B.Cu") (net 14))
 (segment (start 213.337272 34.80441) (end 211.786967 34.80441) (width 0.25) (layer "F.Cu") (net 15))
 (segment (start 214.057299 34.084383) (end 213.337272 34.80441) (width 0.25) (layer "F.Cu") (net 15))
 (segment (start 214.057299 33.68491) (end 214.057299 34.084383) (width 0.25) (layer "F.Cu") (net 15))
 (via (at 214.057299 33.68491) (size 0.8) (drill 0.4) (layers "F.Cu" "B.Cu") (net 15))
 (segment (start 222.203363 33.95941) (end 222.541967 34.298014) (width 0.25) (layer "B.Cu") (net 15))
 (segment (start 214.057299 33.68491) (end 214.331799 33.95941) (width 0.25) (layer "B.Cu") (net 15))
 (segment (start 214.331799 33.95941) (end 222.203363 33.95941) (width 0.25) (layer "B.Cu") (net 15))
 (segment (start 222.541967 34.298014) (end 222.541967 35.38441) (width 0.25) (layer "B.Cu") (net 15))
 (segment (start 211.786967 36.991111) (end 211.786967 37.34441) (width 0.25) (layer "F.Cu") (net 16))
 (segment (start 215.040709 33.23491) (end 215.040709 33.737369) (width 0.25) (layer "F.Cu") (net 16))
 (segment (start 215.040709 33.737369) (end 211.786967 36.991111) (width 0.25) (layer "F.Cu") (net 16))
 (via (at 215.040709 33.23491) (size 0.8) (drill 0.4) (layers "F.Cu" "B.Cu") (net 16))
 (segment (start 218.99941 30.95941) (end 221.54941 33.50941) (width 0.25) (layer "B.Cu") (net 16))
 (segment (start 215.040709 32.759291) (end 216.84059 30.95941) (width 0.25) (layer "B.Cu") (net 16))
 (segment (start 221.54941 33.50941) (end 222.389759 33.50941) (width 0.25) (layer "B.Cu") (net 16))
 (segment (start 223.041967 34.161618) (end 223.041967 35.38441) (width 0.25) (layer "B.Cu") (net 16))
 (segment (start 216.84059 30.95941) (end 218.99941 30.95941) (width 0.25) (layer "B.Cu") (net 16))
 (segment (start 222.389759 33.50941) (end 223.041967 34.161618) (width 0.25) (layer "B.Cu") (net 16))
 (segment (start 215.040709 33.23491) (end 215.040709 32.759291) (width 0.25) (layer "B.Cu") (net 16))
 (segment (start 211.786967 44.96441) (end 217.481058 44.96441) (width 0.4) (layer "F.Cu") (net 1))
 (segment (start 209.11559 46.28441) (end 210.43559 44.96441) (width 0.4) (layer "F.Cu") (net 1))
 (segment (start 210.43559 44.96441) (end 211.786967 44.96441) (width 0.4) (layer "F.Cu") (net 1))
 (segment (start 208.291967 46.28441) (end 209.11559 46.28441) (width 0.4) (layer "F.Cu") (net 1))
 (segment (start 217.481058 44.96441) (end 218.408058 45.89141) (width 0.4) (layer "F.Cu") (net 1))
 (segment (start 219.63559 40.03441) (end 218.771967 40.898033) (width 0.25) (layer "B.Cu") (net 1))
 (segment (start 218.771967 40.898033) (end 218.771967 45.91741) (width 0.25) (layer "B.Cu") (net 1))
 (segment (start 220.141967 40.03441) (end 219.63559 40.03441) (width 0.25) (layer "B.Cu") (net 1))
 (segment (start 213.941967 40.03441) (end 220.141967 40.03441) (width 0.25) (layer "B.Cu") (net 1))
 (segment (start 225.27692 40.602454) (end 224.850876 40.17641) (width 0.4) (layer "B.Cu") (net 6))
 (segment (start 228.08941 46.76941) (end 225.27692 43.95692) (width 0.4) (layer "B.Cu") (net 6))
 (segment (start 232.28059 46.76941) (end 228.08941 46.76941) (width 0.4) (layer "B.Cu") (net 6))
 (segment (start 233.041967 45.61941) (end 233.041967 46.008033) (width 0.4) (layer "B.Cu") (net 6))
 (segment (start 225.27692 43.95692) (end 225.27692 40.602454) (width 0.4) (layer "B.Cu") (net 6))
 (segment (start 233.041967 46.008033) (end 232.28059 46.76941) (width 0.4) (layer "B.Cu") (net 6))
 (segment (start 221.311967 44.581967) (end 221.311967 45.91741) (width 0.25) (layer "B.Cu") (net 2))
 (segment (start 220.46441 43.73441) (end 221.311967 44.581967) (width 0.25) (layer "B.Cu") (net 2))
 (segment (start 220.141967 43.73441) (end 220.46441 43.73441) (width 0.25) (layer "B.Cu") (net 2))
 (segment (start 234.541967 45.61941) (end 234.541967 46.01941) (width 0.4) (layer "B.Cu") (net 5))
 (segment (start 209.147557 49.14) (end 208.291967 48.28441) (width 0.4) (layer "B.Cu") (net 5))
 (segment (start 231.421377 49.14) (end 209.147557 49.14) (width 0.4) (layer "B.Cu") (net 5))
 (segment (start 234.541967 46.01941) (end 231.421377 49.14) (width 0.4) (layer "B.Cu") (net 5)))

